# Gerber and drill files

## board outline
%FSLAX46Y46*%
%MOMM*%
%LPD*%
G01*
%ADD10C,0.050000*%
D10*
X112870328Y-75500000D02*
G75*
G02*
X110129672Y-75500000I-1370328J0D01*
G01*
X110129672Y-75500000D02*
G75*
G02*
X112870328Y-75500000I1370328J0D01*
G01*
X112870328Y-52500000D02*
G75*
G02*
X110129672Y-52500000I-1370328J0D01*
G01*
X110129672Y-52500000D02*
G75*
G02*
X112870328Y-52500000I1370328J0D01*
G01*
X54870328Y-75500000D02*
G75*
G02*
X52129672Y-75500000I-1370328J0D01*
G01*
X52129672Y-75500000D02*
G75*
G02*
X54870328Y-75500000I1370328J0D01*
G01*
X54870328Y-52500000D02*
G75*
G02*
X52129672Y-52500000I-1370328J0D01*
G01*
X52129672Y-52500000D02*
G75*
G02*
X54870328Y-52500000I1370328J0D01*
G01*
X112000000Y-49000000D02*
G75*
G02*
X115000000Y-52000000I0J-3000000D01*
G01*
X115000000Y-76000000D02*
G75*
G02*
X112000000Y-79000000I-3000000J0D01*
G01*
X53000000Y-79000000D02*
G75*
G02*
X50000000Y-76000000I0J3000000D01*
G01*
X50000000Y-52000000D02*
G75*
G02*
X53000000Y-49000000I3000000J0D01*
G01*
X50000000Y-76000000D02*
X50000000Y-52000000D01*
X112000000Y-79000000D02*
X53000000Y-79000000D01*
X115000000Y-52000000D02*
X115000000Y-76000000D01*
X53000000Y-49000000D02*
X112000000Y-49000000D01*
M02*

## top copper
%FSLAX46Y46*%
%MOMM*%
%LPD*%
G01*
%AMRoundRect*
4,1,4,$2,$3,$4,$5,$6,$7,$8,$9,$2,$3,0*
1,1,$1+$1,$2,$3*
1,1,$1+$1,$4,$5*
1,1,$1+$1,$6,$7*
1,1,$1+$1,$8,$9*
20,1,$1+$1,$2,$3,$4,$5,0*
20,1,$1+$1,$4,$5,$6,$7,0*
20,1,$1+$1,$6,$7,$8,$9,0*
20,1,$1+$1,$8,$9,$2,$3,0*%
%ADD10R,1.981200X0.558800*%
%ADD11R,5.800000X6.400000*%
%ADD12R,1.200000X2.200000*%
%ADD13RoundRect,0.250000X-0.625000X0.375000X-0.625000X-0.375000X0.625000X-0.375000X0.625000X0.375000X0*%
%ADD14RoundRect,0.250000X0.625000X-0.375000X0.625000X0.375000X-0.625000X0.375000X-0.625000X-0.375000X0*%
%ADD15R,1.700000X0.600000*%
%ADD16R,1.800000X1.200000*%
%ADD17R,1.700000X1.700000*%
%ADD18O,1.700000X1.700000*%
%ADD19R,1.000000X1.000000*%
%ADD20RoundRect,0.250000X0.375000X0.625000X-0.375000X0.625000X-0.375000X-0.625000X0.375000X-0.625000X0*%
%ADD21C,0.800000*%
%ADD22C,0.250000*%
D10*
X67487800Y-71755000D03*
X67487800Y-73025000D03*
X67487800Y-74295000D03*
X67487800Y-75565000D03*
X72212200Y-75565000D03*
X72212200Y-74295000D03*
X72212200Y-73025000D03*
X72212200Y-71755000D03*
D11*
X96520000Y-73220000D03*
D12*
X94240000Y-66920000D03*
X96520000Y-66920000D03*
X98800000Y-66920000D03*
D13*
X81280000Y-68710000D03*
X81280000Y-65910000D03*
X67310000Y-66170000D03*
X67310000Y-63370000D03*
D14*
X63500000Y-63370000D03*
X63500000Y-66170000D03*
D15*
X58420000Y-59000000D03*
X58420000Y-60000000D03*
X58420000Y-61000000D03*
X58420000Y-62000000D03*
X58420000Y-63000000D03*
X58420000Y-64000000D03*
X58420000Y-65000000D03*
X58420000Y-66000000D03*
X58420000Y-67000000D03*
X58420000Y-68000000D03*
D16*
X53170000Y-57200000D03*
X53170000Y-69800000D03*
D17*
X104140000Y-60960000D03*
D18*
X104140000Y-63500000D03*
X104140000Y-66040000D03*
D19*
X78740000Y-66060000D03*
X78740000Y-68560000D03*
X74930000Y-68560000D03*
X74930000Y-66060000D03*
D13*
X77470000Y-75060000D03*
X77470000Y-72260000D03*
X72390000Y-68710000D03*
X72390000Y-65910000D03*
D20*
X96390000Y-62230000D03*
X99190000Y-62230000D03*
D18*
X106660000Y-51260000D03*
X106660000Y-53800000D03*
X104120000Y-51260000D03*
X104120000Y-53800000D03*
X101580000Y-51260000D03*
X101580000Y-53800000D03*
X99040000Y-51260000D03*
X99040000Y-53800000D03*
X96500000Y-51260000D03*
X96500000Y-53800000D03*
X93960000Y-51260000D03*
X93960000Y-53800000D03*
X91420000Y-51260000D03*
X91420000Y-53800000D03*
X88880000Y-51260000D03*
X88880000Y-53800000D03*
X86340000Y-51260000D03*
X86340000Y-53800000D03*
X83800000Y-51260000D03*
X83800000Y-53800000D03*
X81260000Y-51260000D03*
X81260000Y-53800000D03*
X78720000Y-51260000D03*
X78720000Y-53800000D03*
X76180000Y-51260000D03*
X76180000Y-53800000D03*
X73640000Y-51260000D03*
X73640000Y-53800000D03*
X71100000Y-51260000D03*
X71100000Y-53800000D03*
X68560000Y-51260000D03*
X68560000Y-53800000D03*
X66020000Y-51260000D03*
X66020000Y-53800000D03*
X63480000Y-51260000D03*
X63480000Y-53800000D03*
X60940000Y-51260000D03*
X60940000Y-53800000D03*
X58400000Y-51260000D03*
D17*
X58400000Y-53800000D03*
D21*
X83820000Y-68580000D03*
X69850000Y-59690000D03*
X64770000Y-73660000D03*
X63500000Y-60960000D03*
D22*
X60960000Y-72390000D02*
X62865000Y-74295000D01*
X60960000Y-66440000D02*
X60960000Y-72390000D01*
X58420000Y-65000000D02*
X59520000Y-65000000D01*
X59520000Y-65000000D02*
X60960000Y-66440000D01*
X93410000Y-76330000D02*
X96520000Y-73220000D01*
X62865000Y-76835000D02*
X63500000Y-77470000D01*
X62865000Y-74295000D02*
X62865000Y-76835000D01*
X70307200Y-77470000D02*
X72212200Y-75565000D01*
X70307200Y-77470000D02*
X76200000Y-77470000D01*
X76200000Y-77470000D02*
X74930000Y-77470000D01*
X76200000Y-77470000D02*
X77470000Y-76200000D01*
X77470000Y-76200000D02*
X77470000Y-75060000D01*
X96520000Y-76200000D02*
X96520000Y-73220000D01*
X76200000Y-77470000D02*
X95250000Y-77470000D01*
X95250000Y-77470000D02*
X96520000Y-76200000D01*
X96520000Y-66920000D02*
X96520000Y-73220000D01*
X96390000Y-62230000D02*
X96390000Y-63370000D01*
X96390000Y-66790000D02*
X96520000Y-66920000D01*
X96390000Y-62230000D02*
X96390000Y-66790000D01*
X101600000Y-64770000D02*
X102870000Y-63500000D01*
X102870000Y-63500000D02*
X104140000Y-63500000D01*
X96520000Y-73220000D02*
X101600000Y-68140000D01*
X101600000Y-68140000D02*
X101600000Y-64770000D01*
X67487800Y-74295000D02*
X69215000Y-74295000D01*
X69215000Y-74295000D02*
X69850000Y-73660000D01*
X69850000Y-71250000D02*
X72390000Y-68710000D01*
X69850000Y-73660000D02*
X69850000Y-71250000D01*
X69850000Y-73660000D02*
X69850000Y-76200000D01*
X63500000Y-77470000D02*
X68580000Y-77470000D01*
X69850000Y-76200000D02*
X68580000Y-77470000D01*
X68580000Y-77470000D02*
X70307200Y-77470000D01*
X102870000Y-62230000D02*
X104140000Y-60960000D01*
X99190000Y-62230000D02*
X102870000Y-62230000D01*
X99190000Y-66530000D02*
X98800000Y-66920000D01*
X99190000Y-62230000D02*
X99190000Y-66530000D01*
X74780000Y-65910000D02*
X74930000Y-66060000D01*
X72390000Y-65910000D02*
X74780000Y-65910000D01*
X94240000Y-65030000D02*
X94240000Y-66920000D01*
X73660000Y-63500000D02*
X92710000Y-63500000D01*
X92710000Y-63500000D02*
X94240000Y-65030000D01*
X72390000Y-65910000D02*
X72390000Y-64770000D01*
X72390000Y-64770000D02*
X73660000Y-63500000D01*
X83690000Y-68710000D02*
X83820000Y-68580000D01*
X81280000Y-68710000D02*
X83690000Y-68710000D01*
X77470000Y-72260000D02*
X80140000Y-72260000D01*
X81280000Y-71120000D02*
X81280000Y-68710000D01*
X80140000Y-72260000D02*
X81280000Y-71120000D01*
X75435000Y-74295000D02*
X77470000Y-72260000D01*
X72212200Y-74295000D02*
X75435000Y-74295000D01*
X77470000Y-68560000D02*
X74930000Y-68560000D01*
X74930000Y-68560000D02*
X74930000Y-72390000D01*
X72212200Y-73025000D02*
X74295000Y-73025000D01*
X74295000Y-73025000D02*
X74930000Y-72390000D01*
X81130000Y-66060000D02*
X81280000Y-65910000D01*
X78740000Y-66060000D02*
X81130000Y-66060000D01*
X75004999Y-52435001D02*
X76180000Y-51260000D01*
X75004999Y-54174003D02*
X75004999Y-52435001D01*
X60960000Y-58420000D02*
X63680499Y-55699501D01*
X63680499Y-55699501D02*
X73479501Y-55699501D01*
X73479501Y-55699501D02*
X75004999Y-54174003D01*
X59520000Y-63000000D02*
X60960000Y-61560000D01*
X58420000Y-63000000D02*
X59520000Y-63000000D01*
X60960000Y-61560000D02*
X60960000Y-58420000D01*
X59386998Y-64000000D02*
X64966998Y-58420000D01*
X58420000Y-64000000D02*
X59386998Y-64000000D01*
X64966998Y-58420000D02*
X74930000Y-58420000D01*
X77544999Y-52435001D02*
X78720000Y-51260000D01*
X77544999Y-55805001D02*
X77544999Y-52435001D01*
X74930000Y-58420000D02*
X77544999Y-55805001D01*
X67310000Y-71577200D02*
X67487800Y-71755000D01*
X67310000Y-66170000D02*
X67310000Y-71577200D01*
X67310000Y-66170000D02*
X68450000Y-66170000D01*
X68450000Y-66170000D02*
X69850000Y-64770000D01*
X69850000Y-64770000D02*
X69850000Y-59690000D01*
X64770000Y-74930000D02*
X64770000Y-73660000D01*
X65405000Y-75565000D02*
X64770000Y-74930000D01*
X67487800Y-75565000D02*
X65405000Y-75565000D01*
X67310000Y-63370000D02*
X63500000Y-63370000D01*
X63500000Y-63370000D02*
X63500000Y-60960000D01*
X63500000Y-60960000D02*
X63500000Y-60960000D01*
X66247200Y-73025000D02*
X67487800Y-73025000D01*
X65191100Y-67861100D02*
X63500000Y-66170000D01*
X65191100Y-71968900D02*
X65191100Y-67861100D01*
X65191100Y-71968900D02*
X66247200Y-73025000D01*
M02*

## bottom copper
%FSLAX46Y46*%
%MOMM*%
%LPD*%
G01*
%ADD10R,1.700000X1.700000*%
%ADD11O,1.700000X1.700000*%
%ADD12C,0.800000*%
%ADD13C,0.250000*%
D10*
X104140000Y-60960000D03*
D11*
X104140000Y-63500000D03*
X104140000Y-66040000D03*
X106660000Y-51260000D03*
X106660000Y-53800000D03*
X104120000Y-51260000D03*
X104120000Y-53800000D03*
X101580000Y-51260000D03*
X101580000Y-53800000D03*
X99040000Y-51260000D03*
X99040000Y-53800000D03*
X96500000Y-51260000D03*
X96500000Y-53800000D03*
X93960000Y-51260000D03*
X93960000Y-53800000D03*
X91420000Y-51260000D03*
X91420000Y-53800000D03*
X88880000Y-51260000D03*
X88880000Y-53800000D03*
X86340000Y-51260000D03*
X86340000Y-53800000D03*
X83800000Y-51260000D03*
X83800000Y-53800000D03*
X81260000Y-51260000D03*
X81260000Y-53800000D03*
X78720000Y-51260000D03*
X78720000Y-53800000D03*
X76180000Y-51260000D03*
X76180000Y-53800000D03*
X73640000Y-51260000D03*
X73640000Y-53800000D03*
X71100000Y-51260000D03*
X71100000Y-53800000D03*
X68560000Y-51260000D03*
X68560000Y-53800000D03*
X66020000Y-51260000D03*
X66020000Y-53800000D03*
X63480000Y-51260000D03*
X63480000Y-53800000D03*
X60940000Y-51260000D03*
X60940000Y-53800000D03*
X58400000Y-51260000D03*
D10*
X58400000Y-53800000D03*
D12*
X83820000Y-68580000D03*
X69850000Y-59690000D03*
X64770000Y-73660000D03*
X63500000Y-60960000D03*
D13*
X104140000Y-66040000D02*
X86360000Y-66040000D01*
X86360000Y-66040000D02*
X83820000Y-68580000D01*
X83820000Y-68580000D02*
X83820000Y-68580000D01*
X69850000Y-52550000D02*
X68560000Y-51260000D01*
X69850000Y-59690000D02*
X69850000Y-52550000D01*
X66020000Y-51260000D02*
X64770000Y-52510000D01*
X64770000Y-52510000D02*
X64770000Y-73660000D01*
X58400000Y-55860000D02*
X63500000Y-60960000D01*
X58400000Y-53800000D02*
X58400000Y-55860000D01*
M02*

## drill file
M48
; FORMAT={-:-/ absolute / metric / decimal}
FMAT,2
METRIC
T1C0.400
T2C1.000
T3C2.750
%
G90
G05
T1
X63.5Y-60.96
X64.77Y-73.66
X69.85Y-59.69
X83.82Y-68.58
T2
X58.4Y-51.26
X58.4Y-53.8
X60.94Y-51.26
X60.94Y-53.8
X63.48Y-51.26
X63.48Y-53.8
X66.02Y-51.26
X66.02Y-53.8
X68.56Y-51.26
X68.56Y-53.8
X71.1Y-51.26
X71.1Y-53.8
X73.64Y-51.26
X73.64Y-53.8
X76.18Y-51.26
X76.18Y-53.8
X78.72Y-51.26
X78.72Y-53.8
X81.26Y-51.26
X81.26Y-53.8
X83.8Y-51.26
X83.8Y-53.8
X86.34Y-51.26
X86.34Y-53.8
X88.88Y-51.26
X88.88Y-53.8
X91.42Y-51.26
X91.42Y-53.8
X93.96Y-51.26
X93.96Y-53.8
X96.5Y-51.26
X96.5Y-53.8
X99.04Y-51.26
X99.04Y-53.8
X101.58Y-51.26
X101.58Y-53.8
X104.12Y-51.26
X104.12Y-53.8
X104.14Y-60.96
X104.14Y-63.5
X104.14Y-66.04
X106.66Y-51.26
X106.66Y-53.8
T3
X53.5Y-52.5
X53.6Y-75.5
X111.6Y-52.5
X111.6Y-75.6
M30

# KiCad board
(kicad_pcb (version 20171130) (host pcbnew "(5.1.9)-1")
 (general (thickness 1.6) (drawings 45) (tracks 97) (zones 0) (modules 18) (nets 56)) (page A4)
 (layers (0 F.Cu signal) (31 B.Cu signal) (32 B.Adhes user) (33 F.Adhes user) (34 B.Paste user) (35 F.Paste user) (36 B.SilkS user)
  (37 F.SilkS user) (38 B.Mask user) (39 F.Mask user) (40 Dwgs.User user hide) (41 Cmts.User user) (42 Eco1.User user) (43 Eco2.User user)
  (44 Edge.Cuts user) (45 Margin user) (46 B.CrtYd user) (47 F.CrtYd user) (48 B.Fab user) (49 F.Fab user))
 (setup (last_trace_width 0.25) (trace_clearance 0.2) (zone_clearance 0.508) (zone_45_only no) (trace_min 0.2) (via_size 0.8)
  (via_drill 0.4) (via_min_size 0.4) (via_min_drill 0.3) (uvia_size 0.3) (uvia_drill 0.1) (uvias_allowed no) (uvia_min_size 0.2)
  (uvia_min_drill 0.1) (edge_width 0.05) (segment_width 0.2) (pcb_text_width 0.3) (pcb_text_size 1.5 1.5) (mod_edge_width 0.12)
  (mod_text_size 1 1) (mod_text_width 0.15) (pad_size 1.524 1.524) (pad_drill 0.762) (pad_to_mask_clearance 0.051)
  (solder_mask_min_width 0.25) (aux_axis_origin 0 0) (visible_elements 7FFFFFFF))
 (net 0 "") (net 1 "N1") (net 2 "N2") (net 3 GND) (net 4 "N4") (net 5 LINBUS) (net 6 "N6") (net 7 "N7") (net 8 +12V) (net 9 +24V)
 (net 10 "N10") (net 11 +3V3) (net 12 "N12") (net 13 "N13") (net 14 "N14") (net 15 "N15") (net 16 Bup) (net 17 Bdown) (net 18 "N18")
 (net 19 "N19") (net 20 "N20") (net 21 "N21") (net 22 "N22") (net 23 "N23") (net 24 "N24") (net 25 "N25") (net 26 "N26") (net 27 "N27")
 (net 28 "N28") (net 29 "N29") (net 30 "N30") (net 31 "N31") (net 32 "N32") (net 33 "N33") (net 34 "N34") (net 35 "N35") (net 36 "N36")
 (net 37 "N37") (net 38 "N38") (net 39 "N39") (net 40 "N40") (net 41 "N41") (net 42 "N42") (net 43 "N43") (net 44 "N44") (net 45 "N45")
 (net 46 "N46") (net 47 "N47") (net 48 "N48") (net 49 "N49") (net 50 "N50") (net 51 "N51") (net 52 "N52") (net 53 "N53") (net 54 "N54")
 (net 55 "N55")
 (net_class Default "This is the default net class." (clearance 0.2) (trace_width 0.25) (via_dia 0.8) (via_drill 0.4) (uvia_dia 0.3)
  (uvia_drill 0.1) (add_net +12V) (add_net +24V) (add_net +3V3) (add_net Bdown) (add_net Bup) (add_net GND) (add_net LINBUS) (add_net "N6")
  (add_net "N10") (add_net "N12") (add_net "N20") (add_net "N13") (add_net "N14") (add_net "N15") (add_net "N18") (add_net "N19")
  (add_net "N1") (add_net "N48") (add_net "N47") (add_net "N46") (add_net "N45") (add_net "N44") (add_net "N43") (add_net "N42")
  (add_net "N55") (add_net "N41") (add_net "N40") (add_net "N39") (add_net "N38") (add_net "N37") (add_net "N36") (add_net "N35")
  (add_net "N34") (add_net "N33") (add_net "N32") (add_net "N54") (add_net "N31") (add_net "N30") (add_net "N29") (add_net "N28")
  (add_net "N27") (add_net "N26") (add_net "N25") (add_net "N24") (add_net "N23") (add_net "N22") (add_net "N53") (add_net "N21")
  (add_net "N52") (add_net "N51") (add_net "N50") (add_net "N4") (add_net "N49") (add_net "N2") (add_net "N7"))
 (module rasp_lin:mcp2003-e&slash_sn (layer F.Cu) (at 69.85 73.66)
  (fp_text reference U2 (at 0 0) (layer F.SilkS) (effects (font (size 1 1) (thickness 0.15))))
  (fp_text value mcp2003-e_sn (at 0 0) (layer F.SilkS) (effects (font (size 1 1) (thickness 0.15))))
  (pad 1 smd rect (at -2.3622 -1.905) (size 1.9812 0.5588) (layers F.Cu F.Paste F.Mask) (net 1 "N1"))
  (pad 2 smd rect (at -2.3622 -0.635) (size 1.9812 0.5588) (layers F.Cu F.Paste F.Mask) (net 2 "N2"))
  (pad 3 smd rect (at -2.3622 0.635) (size 1.9812 0.5588) (layers F.Cu F.Paste F.Mask) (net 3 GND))
  (pad 4 smd rect (at -2.3622 1.905) (size 1.9812 0.5588) (layers F.Cu F.Paste F.Mask) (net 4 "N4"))
  (pad 5 smd rect (at 2.3622 1.905) (size 1.9812 0.5588) (layers F.Cu F.Paste F.Mask) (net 3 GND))
  (pad 6 smd rect (at 2.3622 0.635) (size 1.9812 0.5588) (layers F.Cu F.Paste F.Mask) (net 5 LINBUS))
  (pad 7 smd rect (at 2.3622 -0.635) (size 1.9812 0.5588) (layers F.Cu F.Paste F.Mask) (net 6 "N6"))
  (pad 8 smd rect (at 2.3622 -1.905) (size 1.9812 0.5588) (layers F.Cu F.Paste F.Mask) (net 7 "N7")))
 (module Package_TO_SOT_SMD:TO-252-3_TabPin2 (layer F.Cu) (at 96.52 71.12 270)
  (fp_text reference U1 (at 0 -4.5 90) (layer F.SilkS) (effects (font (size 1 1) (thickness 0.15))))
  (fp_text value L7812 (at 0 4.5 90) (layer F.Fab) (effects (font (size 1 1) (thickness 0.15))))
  (pad "" smd rect (at 0.425 1.525 270) (size 3.05 2.75) (layers F.Paste))
  (pad "" smd rect (at 3.775 -1.525 270) (size 3.05 2.75) (layers F.Paste))
  (pad "" smd rect (at 0.425 -1.525 270) (size 3.05 2.75) (layers F.Paste))
  (pad "" smd rect (at 3.775 1.525 270) (size 3.05 2.75) (layers F.Paste))
  (pad 2 smd rect (at 2.1 0 270) (size 6.4 5.8) (layers F.Cu F.Mask) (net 3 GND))
  (pad 3 smd rect (at -4.2 2.28 270) (size 2.2 1.2) (layers F.Cu F.Paste F.Mask) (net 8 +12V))
  (pad 2 smd rect (at -4.2 0 270) (size 2.2 1.2) (layers F.Cu F.Paste F.Mask) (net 3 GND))
  (pad 1 smd rect (at -4.2 -2.28 270) (size 2.2 1.2) (layers F.Cu F.Paste F.Mask) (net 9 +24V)))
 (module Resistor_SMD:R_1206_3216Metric (layer F.Cu) (at 81.28 67.31 270)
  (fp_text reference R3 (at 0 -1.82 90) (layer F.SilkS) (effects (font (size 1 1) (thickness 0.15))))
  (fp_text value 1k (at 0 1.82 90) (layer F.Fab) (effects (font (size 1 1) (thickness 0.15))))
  (pad 2 smd roundrect (at 1.4 0 270) (size 1.25 1.75) (layers F.Cu F.Paste F.Mask) (roundrect_rratio 0.2) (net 5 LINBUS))
  (pad 1 smd roundrect (at -1.4 0 270) (size 1.25 1.75) (layers F.Cu F.Paste F.Mask) (roundrect_rratio 0.2) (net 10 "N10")))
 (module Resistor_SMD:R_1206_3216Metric (layer F.Cu) (at 67.31 64.77 270)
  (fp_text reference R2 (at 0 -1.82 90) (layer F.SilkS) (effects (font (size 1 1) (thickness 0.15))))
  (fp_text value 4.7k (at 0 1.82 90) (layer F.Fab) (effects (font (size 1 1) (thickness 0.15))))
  (pad 2 smd roundrect (at 1.4 0 270) (size 1.25 1.75) (layers F.Cu F.Paste F.Mask) (roundrect_rratio 0.2) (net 1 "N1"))
  (pad 1 smd roundrect (at -1.4 0 270) (size 1.25 1.75) (layers F.Cu F.Paste F.Mask) (roundrect_rratio 0.2) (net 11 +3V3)))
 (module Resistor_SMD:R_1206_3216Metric (layer F.Cu) (at 63.5 64.77 90)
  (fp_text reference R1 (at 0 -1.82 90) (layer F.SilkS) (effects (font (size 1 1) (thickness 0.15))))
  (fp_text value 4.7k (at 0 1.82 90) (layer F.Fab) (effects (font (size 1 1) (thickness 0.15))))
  (pad 2 smd roundrect (at 1.4 0 90) (size 1.25 1.75) (layers F.Cu F.Paste F.Mask) (roundrect_rratio 0.2) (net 11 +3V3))
  (pad 1 smd roundrect (at -1.4 0 90) (size 1.25 1.75) (layers F.Cu F.Paste F.Mask) (roundrect_rratio 0.2) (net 2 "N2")))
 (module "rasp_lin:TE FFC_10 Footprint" (layer F.Cu) (at 58.42 63.5 270)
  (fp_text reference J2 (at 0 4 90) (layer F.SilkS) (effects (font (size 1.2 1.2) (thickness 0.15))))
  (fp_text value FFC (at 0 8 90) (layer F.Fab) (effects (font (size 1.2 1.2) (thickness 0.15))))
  (pad 1 smd rect (at -4.5 0 270) (size 0.6 1.7) (layers F.Cu F.Paste F.Mask) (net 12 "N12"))
  (pad 2 smd rect (at -3.5 0 270) (size 0.6 1.7) (layers F.Cu F.Paste F.Mask) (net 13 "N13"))
  (pad 3 smd rect (at -2.5 0 270) (size 0.6 1.7) (layers F.Cu F.Paste F.Mask) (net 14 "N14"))
  (pad 4 smd rect (at -1.5 0 270) (size 0.6 1.7) (layers F.Cu F.Paste F.Mask) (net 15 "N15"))
  (pad 5 smd rect (at -0.5 0 270) (size 0.6 1.7) (layers F.Cu F.Paste F.Mask) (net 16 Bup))
  (pad 6 smd rect (at 0.5 0 270) (size 0.6 1.7) (layers F.Cu F.Paste F.Mask) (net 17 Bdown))
  (pad 7 smd rect (at 1.5 0 270) (size 0.6 1.7) (layers F.Cu F.Paste F.Mask) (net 3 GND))
  (pad 8 smd rect (at 2.5 0 270) (size 0.6 1.7) (layers F.Cu F.Paste F.Mask) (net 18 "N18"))
  (pad 9 smd rect (at 3.5 0 270) (size 0.6 1.7) (layers F.Cu F.Paste F.Mask) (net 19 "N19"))
  (pad 10 smd rect (at 4.5 0 270) (size 0.6 1.7) (layers F.Cu F.Paste F.Mask) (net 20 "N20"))
  (pad 0 smd rect (at -6.3 5.25 270) (size 1.2 1.8) (layers F.Cu F.Paste F.Mask))
  (pad 0 smd rect (at 6.3 5.25 270) (size 1.2 1.8) (layers F.Cu F.Paste F.Mask)))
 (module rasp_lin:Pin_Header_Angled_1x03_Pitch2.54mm (layer F.Cu) (at 104.14 60.96)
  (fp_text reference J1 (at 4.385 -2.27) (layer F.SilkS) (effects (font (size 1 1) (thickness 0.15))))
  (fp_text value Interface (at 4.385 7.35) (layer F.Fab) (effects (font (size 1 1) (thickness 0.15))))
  (pad 1 thru_hole rect (at 0 0) (size 1.7 1.7) (drill 1) (layers *.Cu *.Mask) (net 9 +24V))
  (pad 2 thru_hole oval (at 0 2.54) (size 1.7 1.7) (drill 1) (layers *.Cu *.Mask) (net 3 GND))
  (pad 3 thru_hole oval (at 0 5.08) (size 1.7 1.7) (drill 1) (layers *.Cu *.Mask) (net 5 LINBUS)))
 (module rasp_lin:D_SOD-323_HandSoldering (layer F.Cu) (at 78.74 67.31 270)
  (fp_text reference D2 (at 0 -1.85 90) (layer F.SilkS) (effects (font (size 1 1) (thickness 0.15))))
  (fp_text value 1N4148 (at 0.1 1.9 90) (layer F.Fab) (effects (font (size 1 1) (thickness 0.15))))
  (pad 1 smd rect (at -1.25 0 270) (size 1 1) (layers F.Cu F.Paste F.Mask) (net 10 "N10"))
  (pad 2 smd rect (at 1.25 0 270) (size 1 1) (layers F.Cu F.Paste F.Mask) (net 6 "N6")))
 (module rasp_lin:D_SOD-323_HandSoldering (layer F.Cu) (at 74.93 67.31 90)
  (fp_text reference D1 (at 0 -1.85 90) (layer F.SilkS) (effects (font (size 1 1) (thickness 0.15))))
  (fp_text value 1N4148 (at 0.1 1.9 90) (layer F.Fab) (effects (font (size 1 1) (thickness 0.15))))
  (pad 1 smd rect (at -1.25 0 90) (size 1 1) (layers F.Cu F.Paste F.Mask) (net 6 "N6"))
  (pad 2 smd rect (at 1.25 0 90) (size 1 1) (layers F.Cu F.Paste F.Mask) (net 8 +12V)))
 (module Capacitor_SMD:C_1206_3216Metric (layer F.Cu) (at 77.47 73.66 270)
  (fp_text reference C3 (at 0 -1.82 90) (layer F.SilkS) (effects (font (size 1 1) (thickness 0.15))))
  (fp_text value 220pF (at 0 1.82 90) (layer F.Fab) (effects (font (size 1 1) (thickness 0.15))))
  (pad 2 smd roundrect (at 1.4 0 270) (size 1.25 1.75) (layers F.Cu F.Paste F.Mask) (roundrect_rratio 0.2) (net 3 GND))
  (pad 1 smd roundrect (at -1.4 0 270) (size 1.25 1.75) (layers F.Cu F.Paste F.Mask) (roundrect_rratio 0.2) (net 5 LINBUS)))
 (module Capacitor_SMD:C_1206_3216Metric (layer F.Cu) (at 72.39 67.31 270)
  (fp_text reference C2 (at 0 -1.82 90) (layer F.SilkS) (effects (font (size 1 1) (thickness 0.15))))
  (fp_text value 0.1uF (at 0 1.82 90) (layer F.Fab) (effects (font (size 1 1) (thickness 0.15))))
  (pad 2 smd roundrect (at 1.4 0 270) (size 1.25 1.75) (layers F.Cu F.Paste F.Mask) (roundrect_rratio 0.2) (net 3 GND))
  (pad 1 smd roundrect (at -1.4 0 270) (size 1.25 1.75) (layers F.Cu F.Paste F.Mask) (roundrect_rratio 0.2) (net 8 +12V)))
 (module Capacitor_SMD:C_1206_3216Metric (layer F.Cu) (at 97.79 62.23 180)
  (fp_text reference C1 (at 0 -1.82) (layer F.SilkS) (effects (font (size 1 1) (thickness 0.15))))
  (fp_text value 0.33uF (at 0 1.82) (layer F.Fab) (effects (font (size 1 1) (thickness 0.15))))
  (pad 2 smd roundrect (at 1.4 0 180) (size 1.25 1.75) (layers F.Cu F.Paste F.Mask) (roundrect_rratio 0.2) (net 3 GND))
  (pad 1 smd roundrect (at -1.4 0 180) (size 1.25 1.75) (layers F.Cu F.Paste F.Mask) (roundrect_rratio 0.2) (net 9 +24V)))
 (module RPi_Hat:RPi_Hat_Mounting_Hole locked (layer F.Cu) (at 53.5 52.5)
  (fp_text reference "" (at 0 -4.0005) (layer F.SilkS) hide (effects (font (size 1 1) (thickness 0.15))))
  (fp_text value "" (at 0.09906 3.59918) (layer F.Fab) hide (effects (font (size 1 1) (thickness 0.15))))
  (pad "" np_thru_hole circle (at 0 0) (size 2.75 2.75) (drill 2.75) (layers *.Cu *.Mask) (solder_mask_margin 1.725) (clearance 1.725)))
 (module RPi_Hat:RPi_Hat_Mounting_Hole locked (layer F.Cu) (at 53.6 75.5)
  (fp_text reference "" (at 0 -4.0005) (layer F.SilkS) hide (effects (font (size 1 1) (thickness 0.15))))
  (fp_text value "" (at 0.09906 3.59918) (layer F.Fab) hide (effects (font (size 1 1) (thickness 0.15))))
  (pad "" np_thru_hole circle (at 0 0) (size 2.75 2.75) (drill 2.75) (layers *.Cu *.Mask) (solder_mask_margin 1.725) (clearance 1.725)))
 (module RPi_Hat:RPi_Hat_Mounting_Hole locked (layer F.Cu) (at 111.6 75.6)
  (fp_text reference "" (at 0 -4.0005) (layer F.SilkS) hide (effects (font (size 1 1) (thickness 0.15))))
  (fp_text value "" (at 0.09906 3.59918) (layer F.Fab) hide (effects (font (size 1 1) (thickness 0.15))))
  (pad "" np_thru_hole circle (at 0 0) (size 2.75 2.75) (drill 2.75) (layers *.Cu *.Mask) (solder_mask_margin 1.725) (clearance 1.725)))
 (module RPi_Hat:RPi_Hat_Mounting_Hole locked (layer F.Cu) (at 111.6 52.5)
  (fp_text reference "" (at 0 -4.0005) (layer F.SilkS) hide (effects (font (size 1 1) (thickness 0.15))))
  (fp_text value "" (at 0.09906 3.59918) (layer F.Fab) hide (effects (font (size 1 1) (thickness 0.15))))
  (pad "" np_thru_hole circle (at 0 0) (size 2.75 2.75) (drill 2.75) (layers *.Cu *.Mask) (solder_mask_margin 1.725) (clearance 1.725)))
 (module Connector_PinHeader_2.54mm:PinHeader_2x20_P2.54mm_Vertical (layer F.Cu) (at 58.4 53.8 90)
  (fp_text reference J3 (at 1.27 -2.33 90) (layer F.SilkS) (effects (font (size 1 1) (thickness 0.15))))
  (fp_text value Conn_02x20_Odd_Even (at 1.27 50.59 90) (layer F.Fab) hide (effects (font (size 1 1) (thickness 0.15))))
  (pad 40 thru_hole oval (at 2.54 48.26 90) (size 1.7 1.7) (drill 1) (layers *.Cu *.Mask) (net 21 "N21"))
  (pad 39 thru_hole oval (at 0 48.26 90) (size 1.7 1.7) (drill 1) (layers *.Cu *.Mask) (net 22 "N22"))
  (pad 38 thru_hole oval (at 2.54 45.72 90) (size 1.7 1.7) (drill 1) (layers *.Cu *.Mask) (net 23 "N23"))
  (pad 37 thru_hole oval (at 0 45.72 90) (size 1.7 1.7) (drill 1) (layers *.Cu *.Mask) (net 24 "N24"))
  (pad 36 thru_hole oval (at 2.54 43.18 90) (size 1.7 1.7) (drill 1) (layers *.Cu *.Mask) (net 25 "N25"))
  (pad 35 thru_hole oval (at 0 43.18 90) (size 1.7 1.7) (drill 1) (layers *.Cu *.Mask) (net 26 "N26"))
  (pad 34 thru_hole oval (at 2.54 40.64 90) (size 1.7 1.7) (drill 1) (layers *.Cu *.Mask) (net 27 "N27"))
  (pad 33 thru_hole oval (at 0 40.64 90) (size 1.7 1.7) (drill 1) (layers *.Cu *.Mask) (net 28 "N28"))
  (pad 32 thru_hole oval (at 2.54 38.1 90) (size 1.7 1.7) (drill 1) (layers *.Cu *.Mask) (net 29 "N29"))
  (pad 31 thru_hole oval (at 0 38.1 90) (size 1.7 1.7) (drill 1) (layers *.Cu *.Mask) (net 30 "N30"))
  (pad 30 thru_hole oval (at 2.54 35.56 90) (size 1.7 1.7) (drill 1) (layers *.Cu *.Mask) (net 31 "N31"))
  (pad 29 thru_hole oval (at 0 35.56 90) (size 1.7 1.7) (drill 1) (layers *.Cu *.Mask) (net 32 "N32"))
  (pad 28 thru_hole oval (at 2.54 33.02 90) (size 1.7 1.7) (drill 1) (layers *.Cu *.Mask) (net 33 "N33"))
  (pad 27 thru_hole oval (at 0 33.02 90) (size 1.7 1.7) (drill 1) (layers *.Cu *.Mask) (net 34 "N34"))
  (pad 26 thru_hole oval (at 2.54 30.48 90) (size 1.7 1.7) (drill 1) (layers *.Cu *.Mask) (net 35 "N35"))
  (pad 25 thru_hole oval (at 0 30.48 90) (size 1.7 1.7) (drill 1) (layers *.Cu *.Mask) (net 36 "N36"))
  (pad 24 thru_hole oval (at 2.54 27.94 90) (size 1.7 1.7) (drill 1) (layers *.Cu *.Mask) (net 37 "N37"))
  (pad 23 thru_hole oval (at 0 27.94 90) (size 1.7 1.7) (drill 1) (layers *.Cu *.Mask) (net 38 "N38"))
  (pad 22 thru_hole oval (at 2.54 25.4 90) (size 1.7 1.7) (drill 1) (layers *.Cu *.Mask) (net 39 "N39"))
  (pad 21 thru_hole oval (at 0 25.4 90) (size 1.7 1.7) (drill 1) (layers *.Cu *.Mask) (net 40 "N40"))
  (pad 20 thru_hole oval (at 2.54 22.86 90) (size 1.7 1.7) (drill 1) (layers *.Cu *.Mask) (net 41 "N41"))
  (pad 19 thru_hole oval (at 0 22.86 90) (size 1.7 1.7) (drill 1) (layers *.Cu *.Mask) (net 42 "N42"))
  (pad 18 thru_hole oval (at 2.54 20.32 90) (size 1.7 1.7) (drill 1) (layers *.Cu *.Mask) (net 17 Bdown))
  (pad 17 thru_hole oval (at 0 20.32 90) (size 1.7 1.7) (drill 1) (layers *.Cu *.Mask) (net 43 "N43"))
  (pad 16 thru_hole oval (at 2.54 17.78 90) (size 1.7 1.7) (drill 1) (layers *.Cu *.Mask) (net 16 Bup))
  (pad 15 thru_hole oval (at 0 17.78 90) (size 1.7 1.7) (drill 1) (layers *.Cu *.Mask) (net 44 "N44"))
  (pad 14 thru_hole oval (at 2.54 15.24 90) (size 1.7 1.7) (drill 1) (layers *.Cu *.Mask) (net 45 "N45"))
  (pad 13 thru_hole oval (at 0 15.24 90) (size 1.7 1.7) (drill 1) (layers *.Cu *.Mask) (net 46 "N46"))
  (pad 12 thru_hole oval (at 2.54 12.7 90) (size 1.7 1.7) (drill 1) (layers *.Cu *.Mask) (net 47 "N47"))
  (pad 11 thru_hole oval (at 0 12.7 90) (size 1.7 1.7) (drill 1) (layers *.Cu *.Mask) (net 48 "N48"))
  (pad 10 thru_hole oval (at 2.54 10.16 90) (size 1.7 1.7) (drill 1) (layers *.Cu *.Mask) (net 1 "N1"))
  (pad 9 thru_hole oval (at 0 10.16 90) (size 1.7 1.7) (drill 1) (layers *.Cu *.Mask) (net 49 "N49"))
  (pad 8 thru_hole oval (at 2.54 7.62 90) (size 1.7 1.7) (drill 1) (layers *.Cu *.Mask) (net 4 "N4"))
  (pad 7 thru_hole oval (at 0 7.62 90) (size 1.7 1.7) (drill 1) (layers *.Cu *.Mask) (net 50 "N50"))
  (pad 6 thru_hole oval (at 2.54 5.08 90) (size 1.7 1.7) (drill 1) (layers *.Cu *.Mask) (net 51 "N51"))
  (pad 5 thru_hole oval (at 0 5.08 90) (size 1.7 1.7) (drill 1) (layers *.Cu *.Mask) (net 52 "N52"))
  (pad 4 thru_hole oval (at 2.54 2.54 90) (size 1.7 1.7) (drill 1) (layers *.Cu *.Mask) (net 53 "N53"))
  (pad 3 thru_hole oval (at 0 2.54 90) (size 1.7 1.7) (drill 1) (layers *.Cu *.Mask) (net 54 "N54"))
  (pad 2 thru_hole oval (at 2.54 0 90) (size 1.7 1.7) (drill 1) (layers *.Cu *.Mask) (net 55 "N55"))
  (pad 1 thru_hole rect (at 0 0 90) (size 1.7 1.7) (drill 1) (layers *.Cu *.Mask) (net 11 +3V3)))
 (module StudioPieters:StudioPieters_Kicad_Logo (layer F.Cu) (at 202.8 170.6)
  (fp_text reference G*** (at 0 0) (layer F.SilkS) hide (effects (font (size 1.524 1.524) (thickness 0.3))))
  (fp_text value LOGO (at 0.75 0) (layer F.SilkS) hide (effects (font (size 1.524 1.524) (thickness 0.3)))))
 (gr_circle (center 111.5 75.5) (end 111.47 76.87) (layer Edge.Cuts) (width 0.05))
 (gr_circle (center 111.5 52.5) (end 111.47 53.87) (layer Edge.Cuts) (width 0.05))
 (gr_circle (center 53.5 75.5) (end 53.47 76.87) (layer Edge.Cuts) (width 0.05))
 (gr_circle (center 53.5 52.5) (end 53.47 53.87) (layer Edge.Cuts) (width 0.05))
 (gr_arc (start 112 52) (end 115 52) (angle -90) (layer Edge.Cuts) (width 0.05))
 (gr_arc (start 112 76) (end 112 79) (angle -90) (layer Edge.Cuts) (width 0.05))
 (gr_arc (start 53 76) (end 50 76) (angle -90) (layer Edge.Cuts) (width 0.05))
 (gr_arc (start 53 52) (end 53 49) (angle -90) (layer Edge.Cuts) (width 0.05))
 (gr_line (start 50 76) (end 50 52) (layer Edge.Cuts) (width 0.05))
 (gr_line (start 112 79) (end 53 79) (layer Edge.Cuts) (width 0.05))
 (gr_line (start 115 52) (end 115 76) (layer Edge.Cuts) (width 0.05))
 (gr_line (start 53 49) (end 112 49) (layer Edge.Cuts) (width 0.05))
 (segment (start 60.96 72.39) (end 62.865 74.295) (width 0.25) (layer F.Cu) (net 3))
 (segment (start 60.96 66.44) (end 60.96 72.39) (width 0.25) (layer F.Cu) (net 3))
 (segment (start 58.42 65) (end 59.52 65) (width 0.25) (layer F.Cu) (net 3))
 (segment (start 59.52 65) (end 60.96 66.44) (width 0.25) (layer F.Cu) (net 3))
 (segment (start 93.41 76.33) (end 96.52 73.22) (width 0.25) (layer F.Cu) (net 3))
 (segment (start 62.865 76.835) (end 63.5 77.47) (width 0.25) (layer F.Cu) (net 3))
 (segment (start 62.865 74.295) (end 62.865 76.835) (width 0.25) (layer F.Cu) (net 3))
 (segment (start 70.3072 77.47) (end 72.2122 75.565) (width 0.25) (layer F.Cu) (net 3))
 (segment (start 70.3072 77.47) (end 76.2 77.47) (width 0.25) (layer F.Cu) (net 3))
 (segment (start 76.2 77.47) (end 74.93 77.47) (width 0.25) (layer F.Cu) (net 3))
 (segment (start 76.2 77.47) (end 77.47 76.2) (width 0.25) (layer F.Cu) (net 3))
 (segment (start 77.47 76.2) (end 77.47 75.06) (width 0.25) (layer F.Cu) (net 3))
 (segment (start 96.52 76.2) (end 96.52 73.22) (width 0.25) (layer F.Cu) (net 3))
 (segment (start 76.2 77.47) (end 95.25 77.47) (width 0.25) (layer F.Cu) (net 3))
 (segment (start 95.25 77.47) (end 96.52 76.2) (width 0.25) (layer F.Cu) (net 3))
 (segment (start 96.52 66.92) (end 96.52 73.22) (width 0.25) (layer F.Cu) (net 3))
 (segment (start 96.39 62.23) (end 96.39 63.37) (width 0.25) (layer F.Cu) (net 3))
 (segment (start 96.39 66.79) (end 96.52 66.92) (width 0.25) (layer F.Cu) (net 3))
 (segment (start 96.39 62.23) (end 96.39 66.79) (width 0.25) (layer F.Cu) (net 3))
 (segment (start 101.6 64.77) (end 102.87 63.5) (width 0.25) (layer F.Cu) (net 3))
 (segment (start 102.87 63.5) (end 104.14 63.5) (width 0.25) (layer F.Cu) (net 3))
 (segment (start 96.52 73.22) (end 101.6 68.14) (width 0.25) (layer F.Cu) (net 3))
 (segment (start 101.6 68.14) (end 101.6 64.77) (width 0.25) (layer F.Cu) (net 3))
 (segment (start 67.4878 74.295) (end 69.215 74.295) (width 0.25) (layer F.Cu) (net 3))
 (segment (start 69.215 74.295) (end 69.85 73.66) (width 0.25) (layer F.Cu) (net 3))
 (segment (start 69.85 71.25) (end 72.39 68.71) (width 0.25) (layer F.Cu) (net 3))
 (segment (start 69.85 73.66) (end 69.85 71.25) (width 0.25) (layer F.Cu) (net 3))
 (segment (start 69.85 73.66) (end 69.85 76.2) (width 0.25) (layer F.Cu) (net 3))
 (segment (start 63.5 77.47) (end 68.58 77.47) (width 0.25) (layer F.Cu) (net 3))
 (segment (start 69.85 76.2) (end 68.58 77.47) (width 0.25) (layer F.Cu) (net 3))
 (segment (start 68.58 77.47) (end 70.3072 77.47) (width 0.25) (layer F.Cu) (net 3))
 (segment (start 102.87 62.23) (end 104.14 60.96) (width 0.25) (layer F.Cu) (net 9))
 (segment (start 99.19 62.23) (end 102.87 62.23) (width 0.25) (layer F.Cu) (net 9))
 (segment (start 99.19 66.53) (end 98.8 66.92) (width 0.25) (layer F.Cu) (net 9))
 (segment (start 99.19 62.23) (end 99.19 66.53) (width 0.25) (layer F.Cu) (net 9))
 (segment (start 74.78 65.91) (end 74.93 66.06) (width 0.25) (layer F.Cu) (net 8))
 (segment (start 72.39 65.91) (end 74.78 65.91) (width 0.25) (layer F.Cu) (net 8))
 (segment (start 94.24 65.03) (end 94.24 66.92) (width 0.25) (layer F.Cu) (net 8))
 (segment (start 73.66 63.5) (end 92.71 63.5) (width 0.25) (layer F.Cu) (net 8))
 (segment (start 92.71 63.5) (end 94.24 65.03) (width 0.25) (layer F.Cu) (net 8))
 (segment (start 72.39 65.91) (end 72.39 64.77) (width 0.25) (layer F.Cu) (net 8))
 (segment (start 72.39 64.77) (end 73.66 63.5) (width 0.25) (layer F.Cu) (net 8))
 (segment (start 104.14 66.04) (end 86.36 66.04) (width 0.25) (layer B.Cu) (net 5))
 (segment (start 86.36 66.04) (end 83.82 68.58) (width 0.25) (layer B.Cu) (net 5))
 (segment (start 83.82 68.58) (end 83.82 68.58) (width 0.25) (layer B.Cu) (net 5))
 (via (at 83.82 68.58) (size 0.8) (drill 0.4) (layers F.Cu B.Cu) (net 5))
 (segment (start 83.69 68.71) (end 83.82 68.58) (width 0.25) (layer F.Cu) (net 5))
 (segment (start 81.28 68.71) (end 83.69 68.71) (width 0.25) (layer F.Cu) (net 5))
 (segment (start 77.47 72.26) (end 80.14 72.26) (width 0.25) (layer F.Cu) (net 5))
 (segment (start 81.28 71.12) (end 81.28 68.71) (width 0.25) (layer F.Cu) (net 5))
 (segment (start 80.14 72.26) (end 81.28 71.12) (width 0.25) (layer F.Cu) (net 5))
 (segment (start 75.435 74.295) (end 77.47 72.26) (width 0.25) (layer F.Cu) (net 5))
 (segment (start 72.2122 74.295) (end 75.435 74.295) (width 0.25) (layer F.Cu) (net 5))
 (segment (start 77.47 68.56) (end 74.93 68.56) (width 0.25) (layer F.Cu) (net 6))
 (segment (start 74.93 68.56) (end 74.93 72.39) (width 0.25) (layer F.Cu) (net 6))
 (segment (start 72.2122 73.025) (end 74.295 73.025) (width 0.25) (layer F.Cu) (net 6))
 (segment (start 74.295 73.025) (end 74.93 72.39) (width 0.25) (layer F.Cu) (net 6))
 (segment (start 81.13 66.06) (end 81.28 65.91) (width 0.25) (layer F.Cu) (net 10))
 (segment (start 78.74 66.06) (end 81.13 66.06) (width 0.25) (layer F.Cu) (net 10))
 (segment (start 75.004999 52.435001) (end 76.18 51.26) (width 0.25) (layer F.Cu) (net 16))
 (segment (start 75.004999 54.174003) (end 75.004999 52.435001) (width 0.25) (layer F.Cu) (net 16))
 (segment (start 60.96 58.42) (end 63.680499 55.699501) (width 0.25) (layer F.Cu) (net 16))
 (segment (start 63.680499 55.699501) (end 73.479501 55.699501) (width 0.25) (layer F.Cu) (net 16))
 (segment (start 73.479501 55.699501) (end 75.004999 54.174003) (width 0.25) (layer F.Cu) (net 16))
 (segment (start 59.52 63) (end 60.96 61.56) (width 0.25) (layer F.Cu) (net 16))
 (segment (start 58.42 63) (end 59.52 63) (width 0.25) (layer F.Cu) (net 16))
 (segment (start 60.96 61.56) (end 60.96 58.42) (width 0.25) (layer F.Cu) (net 16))
 (segment (start 59.386998 64) (end 64.966998 58.42) (width 0.25) (layer F.Cu) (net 17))
 (segment (start 58.42 64) (end 59.386998 64) (width 0.25) (layer F.Cu) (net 17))
 (segment (start 64.966998 58.42) (end 74.93 58.42) (width 0.25) (layer F.Cu) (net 17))
 (segment (start 77.544999 52.435001) (end 78.72 51.26) (width 0.25) (layer F.Cu) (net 17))
 (segment (start 77.544999 55.805001) (end 77.544999 52.435001) (width 0.25) (layer F.Cu) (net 17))
 (segment (start 74.93 58.42) (end 77.544999 55.805001) (width 0.25) (layer F.Cu) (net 17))
 (segment (start 67.31 71.5772) (end 67.4878 71.755) (width 0.25) (layer F.Cu) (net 1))
 (segment (start 67.31 66.17) (end 67.31 71.5772) (width 0.25) (layer F.Cu) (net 1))
 (segment (start 67.31 66.17) (end 68.45 66.17) (width 0.25) (layer F.Cu) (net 1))
 (segment (start 68.45 66.17) (end 69.85 64.77) (width 0.25) (layer F.Cu) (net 1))
 (segment (start 69.85 64.77) (end 69.85 59.69) (width 0.25) (layer F.Cu) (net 1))
 (via (at 69.85 59.69) (size 0.8) (drill 0.4) (layers F.Cu B.Cu) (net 1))
 (segment (start 69.85 52.55) (end 68.56 51.26) (width 0.25) (layer B.Cu) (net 1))
 (segment (start 69.85 59.69) (end 69.85 52.55) (width 0.25) (layer B.Cu) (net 1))
 (segment (start 66.02 51.26) (end 64.77 52.51) (width 0.25) (layer B.Cu) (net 4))
 (via (at 64.77 73.66) (size 0.8) (drill 0.4) (layers F.Cu B.Cu) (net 4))
 (segment (start 64.77 52.51) (end 64.77 73.66) (width 0.25) (layer B.Cu) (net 4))
 (segment (start 64.77 74.93) (end 64.77 73.66) (width 0.25) (layer F.Cu) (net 4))
 (segment (start 65.405 75.565) (end 64.77 74.93) (width 0.25) (layer F.Cu) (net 4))
 (segment (start 67.4878 75.565) (end 65.405 75.565) (width 0.25) (layer F.Cu) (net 4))
 (segment (start 67.31 63.37) (end 63.5 63.37) (width 0.25) (layer F.Cu) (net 11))
 (segment (start 63.5 63.37) (end 63.5 60.96) (width 0.25) (layer F.Cu) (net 11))
 (segment (start 63.5 60.96) (end 63.5 60.96) (width 0.25) (layer F.Cu) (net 11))
 (via (at 63.5 60.96) (size 0.8) (drill 0.4) (layers F.Cu B.Cu) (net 11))
 (segment (start 58.4 55.86) (end 63.5 60.96) (width 0.25) (layer B.Cu) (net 11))
 (segment (start 58.4 53.8) (end 58.4 55.86) (width 0.25) (layer B.Cu) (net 11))
 (segment (start 66.2472 73.025) (end 67.4878 73.025) (width 0.25) (layer F.Cu) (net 2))
 (segment (start 65.1911 67.8611) (end 63.5 66.17) (width 0.25) (layer F.Cu) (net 2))
 (segment (start 65.1911 71.9689) (end 65.1911 67.8611) (width 0.25) (layer F.Cu) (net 2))
 (segment (start 65.1911 71.9689) (end 66.2472 73.025) (width 0.25) (layer F.Cu) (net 2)))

